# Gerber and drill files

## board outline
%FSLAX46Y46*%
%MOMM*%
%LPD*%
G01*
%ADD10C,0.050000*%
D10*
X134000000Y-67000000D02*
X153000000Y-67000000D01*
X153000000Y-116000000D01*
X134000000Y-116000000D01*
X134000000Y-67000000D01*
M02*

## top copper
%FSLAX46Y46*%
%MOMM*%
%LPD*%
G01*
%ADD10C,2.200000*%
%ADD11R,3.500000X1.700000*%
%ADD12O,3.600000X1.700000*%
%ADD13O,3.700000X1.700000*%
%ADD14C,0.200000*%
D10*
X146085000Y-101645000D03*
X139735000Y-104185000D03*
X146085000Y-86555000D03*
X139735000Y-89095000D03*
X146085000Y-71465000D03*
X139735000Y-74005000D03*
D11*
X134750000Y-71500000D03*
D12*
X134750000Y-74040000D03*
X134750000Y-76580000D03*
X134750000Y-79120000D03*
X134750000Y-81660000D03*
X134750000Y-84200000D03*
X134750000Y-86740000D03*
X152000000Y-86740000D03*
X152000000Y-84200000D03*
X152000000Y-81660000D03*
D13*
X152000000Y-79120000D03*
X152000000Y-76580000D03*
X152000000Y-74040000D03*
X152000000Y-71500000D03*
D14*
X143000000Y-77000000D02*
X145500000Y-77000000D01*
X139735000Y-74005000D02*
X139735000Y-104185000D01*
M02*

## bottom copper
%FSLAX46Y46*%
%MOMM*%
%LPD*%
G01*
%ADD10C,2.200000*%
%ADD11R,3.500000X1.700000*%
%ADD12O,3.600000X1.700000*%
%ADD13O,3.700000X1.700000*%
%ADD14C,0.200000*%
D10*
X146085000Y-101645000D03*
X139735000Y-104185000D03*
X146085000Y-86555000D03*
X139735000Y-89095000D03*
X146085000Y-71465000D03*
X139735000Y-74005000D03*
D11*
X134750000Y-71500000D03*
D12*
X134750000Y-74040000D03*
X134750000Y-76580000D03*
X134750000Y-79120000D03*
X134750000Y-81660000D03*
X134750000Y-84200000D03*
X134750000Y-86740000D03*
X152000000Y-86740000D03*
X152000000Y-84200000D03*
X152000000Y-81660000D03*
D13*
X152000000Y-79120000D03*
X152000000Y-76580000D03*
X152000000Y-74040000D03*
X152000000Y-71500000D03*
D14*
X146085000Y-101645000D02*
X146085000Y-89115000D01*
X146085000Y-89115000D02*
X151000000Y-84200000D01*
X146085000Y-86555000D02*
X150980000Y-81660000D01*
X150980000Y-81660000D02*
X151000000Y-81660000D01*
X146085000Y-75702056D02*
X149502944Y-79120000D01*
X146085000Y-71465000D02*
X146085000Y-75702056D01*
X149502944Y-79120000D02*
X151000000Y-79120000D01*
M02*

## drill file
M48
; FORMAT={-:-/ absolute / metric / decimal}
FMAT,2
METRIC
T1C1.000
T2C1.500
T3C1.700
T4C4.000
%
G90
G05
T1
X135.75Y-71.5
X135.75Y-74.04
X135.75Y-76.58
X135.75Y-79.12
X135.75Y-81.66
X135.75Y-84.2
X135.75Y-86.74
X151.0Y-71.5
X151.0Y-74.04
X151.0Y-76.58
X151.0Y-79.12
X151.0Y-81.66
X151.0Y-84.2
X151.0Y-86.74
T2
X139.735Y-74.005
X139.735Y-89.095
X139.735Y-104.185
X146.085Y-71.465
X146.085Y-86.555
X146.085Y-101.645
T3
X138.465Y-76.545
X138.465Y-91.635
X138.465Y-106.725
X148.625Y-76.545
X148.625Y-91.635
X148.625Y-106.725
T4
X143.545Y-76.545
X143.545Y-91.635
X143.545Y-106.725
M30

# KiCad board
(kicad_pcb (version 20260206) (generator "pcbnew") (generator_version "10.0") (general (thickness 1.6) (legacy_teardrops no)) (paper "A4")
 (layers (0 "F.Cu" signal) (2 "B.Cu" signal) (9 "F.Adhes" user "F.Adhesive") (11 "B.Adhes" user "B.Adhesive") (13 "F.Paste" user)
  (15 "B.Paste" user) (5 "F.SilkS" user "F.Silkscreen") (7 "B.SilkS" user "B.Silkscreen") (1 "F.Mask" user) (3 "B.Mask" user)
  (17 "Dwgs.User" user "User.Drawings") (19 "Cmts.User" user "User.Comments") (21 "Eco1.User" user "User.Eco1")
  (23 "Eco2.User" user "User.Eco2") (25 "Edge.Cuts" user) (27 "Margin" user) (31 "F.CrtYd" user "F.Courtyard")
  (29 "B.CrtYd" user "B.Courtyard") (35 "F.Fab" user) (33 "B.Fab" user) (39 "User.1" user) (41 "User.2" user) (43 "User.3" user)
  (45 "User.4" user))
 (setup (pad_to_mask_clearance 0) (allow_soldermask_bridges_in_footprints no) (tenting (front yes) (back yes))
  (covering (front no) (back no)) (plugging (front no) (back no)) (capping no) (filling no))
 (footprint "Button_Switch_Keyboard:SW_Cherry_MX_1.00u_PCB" (layer "F.Cu") (at 146.085 101.645)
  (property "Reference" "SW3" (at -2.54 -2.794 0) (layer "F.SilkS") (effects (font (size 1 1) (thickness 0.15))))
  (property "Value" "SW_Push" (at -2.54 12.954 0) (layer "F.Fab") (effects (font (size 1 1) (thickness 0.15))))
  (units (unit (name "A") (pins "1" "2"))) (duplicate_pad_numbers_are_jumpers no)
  (pad "" np_thru_hole circle (at -7.62 5.08) (size 1.7 1.7) (drill 1.7) (layers "*.Cu" "*.Mask"))
  (pad "" np_thru_hole circle (at -2.54 5.08) (size 4 4) (drill 4) (layers "*.Cu" "*.Mask"))
  (pad "" np_thru_hole circle (at 2.54 5.08) (size 1.7 1.7) (drill 1.7) (layers "*.Cu" "*.Mask"))
  (pad "1" thru_hole circle (at 0 0) (size 2.2 2.2) (drill 1.5) (layers "*.Cu" "*.Mask") (remove_unused_layers no)
   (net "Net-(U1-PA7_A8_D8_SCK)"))
  (pad "2" thru_hole circle (at -6.35 2.54) (size 2.2 2.2) (drill 1.5) (layers "*.Cu" "*.Mask") (remove_unused_layers no) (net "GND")))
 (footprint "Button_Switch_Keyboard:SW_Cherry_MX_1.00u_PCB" (layer "F.Cu") (at 146.085 86.555)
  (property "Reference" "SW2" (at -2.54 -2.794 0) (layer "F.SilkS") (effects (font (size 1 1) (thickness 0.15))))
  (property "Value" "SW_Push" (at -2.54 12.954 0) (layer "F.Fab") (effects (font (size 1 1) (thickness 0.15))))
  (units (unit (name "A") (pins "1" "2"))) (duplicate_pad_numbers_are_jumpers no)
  (pad "" np_thru_hole circle (at -7.62 5.08) (size 1.7 1.7) (drill 1.7) (layers "*.Cu" "*.Mask"))
  (pad "" np_thru_hole circle (at -2.54 5.08) (size 4 4) (drill 4) (layers "*.Cu" "*.Mask"))
  (pad "" np_thru_hole circle (at 2.54 5.08) (size 1.7 1.7) (drill 1.7) (layers "*.Cu" "*.Mask"))
  (pad "1" thru_hole circle (at 0 0) (size 2.2 2.2) (drill 1.5) (layers "*.Cu" "*.Mask") (remove_unused_layers no)
   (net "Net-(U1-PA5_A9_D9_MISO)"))
  (pad "2" thru_hole circle (at -6.35 2.54) (size 2.2 2.2) (drill 1.5) (layers "*.Cu" "*.Mask") (remove_unused_layers no) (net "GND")))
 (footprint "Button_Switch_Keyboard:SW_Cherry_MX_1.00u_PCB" (layer "F.Cu") (at 146.085 71.465)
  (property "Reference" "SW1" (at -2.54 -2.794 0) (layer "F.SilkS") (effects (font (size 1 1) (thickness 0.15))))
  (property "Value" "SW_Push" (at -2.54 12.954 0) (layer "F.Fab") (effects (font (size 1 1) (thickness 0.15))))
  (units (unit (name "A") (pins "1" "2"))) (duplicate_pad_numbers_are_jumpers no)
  (pad "" np_thru_hole circle (at -7.62 5.08) (size 1.7 1.7) (drill 1.7) (layers "*.Cu" "*.Mask"))
  (pad "" np_thru_hole circle (at -2.54 5.08) (size 4 4) (drill 4) (layers "*.Cu" "*.Mask"))
  (pad "" np_thru_hole circle (at 2.54 5.08) (size 1.7 1.7) (drill 1.7) (layers "*.Cu" "*.Mask"))
  (pad "1" thru_hole circle (at 0 0) (size 2.2 2.2) (drill 1.5) (layers "*.Cu" "*.Mask") (remove_unused_layers no)
   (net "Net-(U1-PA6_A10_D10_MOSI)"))
  (pad "2" thru_hole circle (at -6.35 2.54) (size 2.2 2.2) (drill 1.5) (layers "*.Cu" "*.Mask") (remove_unused_layers no) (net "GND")))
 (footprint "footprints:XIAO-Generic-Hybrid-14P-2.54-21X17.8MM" (layer "F.Cu") (at 143.375 79.12)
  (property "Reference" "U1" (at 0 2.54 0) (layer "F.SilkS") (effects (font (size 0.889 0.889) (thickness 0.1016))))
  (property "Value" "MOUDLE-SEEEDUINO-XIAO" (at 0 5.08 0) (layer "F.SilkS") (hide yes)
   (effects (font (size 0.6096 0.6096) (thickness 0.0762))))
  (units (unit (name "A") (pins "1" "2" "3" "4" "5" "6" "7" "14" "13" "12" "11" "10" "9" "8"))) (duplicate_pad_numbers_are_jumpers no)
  (pad "1" thru_hole rect (at -7.625 -7.62) (size 3.5 1.7) (drill 1 (offset -1 0)) (layers "*.Cu" "*.Mask") (remove_unused_layers no)
   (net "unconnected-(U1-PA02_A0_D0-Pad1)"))
  (pad "2" thru_hole oval (at -7.625 -5.08) (size 3.6 1.7) (drill 1 (offset -1 0)) (layers "*.Cu" "*.Mask") (remove_unused_layers no)
   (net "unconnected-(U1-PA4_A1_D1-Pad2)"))
  (pad "3" thru_hole oval (at -7.625 -2.54) (size 3.6 1.7) (drill 1 (offset -1 0)) (layers "*.Cu" "*.Mask") (remove_unused_layers no)
   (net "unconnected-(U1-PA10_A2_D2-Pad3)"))
  (pad "4" thru_hole oval (at -7.625 0) (size 3.6 1.7) (drill 1 (offset -1 0)) (layers "*.Cu" "*.Mask") (remove_unused_layers no)
   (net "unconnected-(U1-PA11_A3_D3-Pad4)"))
  (pad "5" thru_hole oval (at -7.625 2.54) (size 3.6 1.7) (drill 1 (offset -1 0)) (layers "*.Cu" "*.Mask") (remove_unused_layers no)
   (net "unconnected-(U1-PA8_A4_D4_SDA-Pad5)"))
  (pad "6" thru_hole oval (at -7.625 5.08 180) (size 3.6 1.7) (drill 1 (offset 1 0)) (layers "*.Cu" "*.Mask") (remove_unused_layers no)
   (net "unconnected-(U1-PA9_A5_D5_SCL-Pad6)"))
  (pad "7" thru_hole oval (at -7.625 7.62) (size 3.6 1.7) (drill 1 (offset -1 0)) (layers "*.Cu" "*.Mask") (remove_unused_layers no)
   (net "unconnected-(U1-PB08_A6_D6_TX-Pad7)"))
  (pad "8" thru_hole oval (at 7.625 7.62) (size 3.6 1.7) (drill 1 (offset 1 0)) (layers "*.Cu" "*.Mask") (remove_unused_layers no)
   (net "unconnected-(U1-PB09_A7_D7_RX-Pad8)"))
  (pad "9" thru_hole oval (at 7.625 5.08) (size 3.6 1.7) (drill 1 (offset 1 0)) (layers "*.Cu" "*.Mask") (remove_unused_layers no)
   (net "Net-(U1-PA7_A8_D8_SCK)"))
  (pad "10" thru_hole oval (at 7.625 2.54) (size 3.6 1.7) (drill 1 (offset 1 0)) (layers "*.Cu" "*.Mask") (remove_unused_layers no)
   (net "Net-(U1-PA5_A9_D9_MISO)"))
  (pad "11" thru_hole oval (at 7.625 0) (size 3.7 1.7) (drill 1 (offset 1 0)) (layers "*.Cu" "*.Mask") (remove_unused_layers no)
   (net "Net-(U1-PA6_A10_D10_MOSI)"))
  (pad "12" thru_hole oval (at 7.625 -2.54) (size 3.7 1.7) (drill 1 (offset 1 0)) (layers "*.Cu" "*.Mask") (remove_unused_layers no)
   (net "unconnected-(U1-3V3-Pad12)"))
  (pad "13" thru_hole oval (at 7.625 -5.08) (size 3.7 1.7) (drill 1 (offset 1 0)) (layers "*.Cu" "*.Mask") (remove_unused_layers no)
   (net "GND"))
  (pad "14" thru_hole oval (at 7.625 -7.62) (size 3.7 1.7) (drill 1 (offset 1 0)) (layers "*.Cu" "*.Mask") (remove_unused_layers no)
   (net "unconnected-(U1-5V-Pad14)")))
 (gr_rect (start 134 67) (end 153 116) (stroke (width 0.05) (type default)) (fill no) (layer "Edge.Cuts"))
 (segment (start 143 77) (end 145.5 77) (width 0.2) (layer "F.Cu") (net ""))
 (segment (start 146.085 101.645) (end 146.085 89.115) (width 0.2) (layer "B.Cu") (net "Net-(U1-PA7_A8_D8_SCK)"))
 (segment (start 146.085 89.115) (end 151 84.2) (width 0.2) (layer "B.Cu") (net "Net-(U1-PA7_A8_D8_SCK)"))
 (segment (start 139.735 74.005) (end 139.735 104.185) (width 0.2) (layer "F.Cu") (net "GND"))
 (segment (start 146.085 86.555) (end 150.98 81.66) (width 0.2) (layer "B.Cu") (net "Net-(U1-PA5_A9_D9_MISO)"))
 (segment (start 150.98 81.66) (end 151 81.66) (width 0.2) (layer "B.Cu") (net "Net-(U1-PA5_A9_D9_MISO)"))
 (segment (start 146.085 75.702056) (end 149.502944 79.12) (width 0.2) (layer "B.Cu") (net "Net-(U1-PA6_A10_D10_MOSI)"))
 (segment (start 146.085 71.465) (end 146.085 75.702056) (width 0.2) (layer "B.Cu") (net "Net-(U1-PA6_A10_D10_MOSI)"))
 (segment (start 149.502944 79.12) (end 151 79.12) (width 0.2) (layer "B.Cu") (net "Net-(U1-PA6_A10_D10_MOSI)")))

